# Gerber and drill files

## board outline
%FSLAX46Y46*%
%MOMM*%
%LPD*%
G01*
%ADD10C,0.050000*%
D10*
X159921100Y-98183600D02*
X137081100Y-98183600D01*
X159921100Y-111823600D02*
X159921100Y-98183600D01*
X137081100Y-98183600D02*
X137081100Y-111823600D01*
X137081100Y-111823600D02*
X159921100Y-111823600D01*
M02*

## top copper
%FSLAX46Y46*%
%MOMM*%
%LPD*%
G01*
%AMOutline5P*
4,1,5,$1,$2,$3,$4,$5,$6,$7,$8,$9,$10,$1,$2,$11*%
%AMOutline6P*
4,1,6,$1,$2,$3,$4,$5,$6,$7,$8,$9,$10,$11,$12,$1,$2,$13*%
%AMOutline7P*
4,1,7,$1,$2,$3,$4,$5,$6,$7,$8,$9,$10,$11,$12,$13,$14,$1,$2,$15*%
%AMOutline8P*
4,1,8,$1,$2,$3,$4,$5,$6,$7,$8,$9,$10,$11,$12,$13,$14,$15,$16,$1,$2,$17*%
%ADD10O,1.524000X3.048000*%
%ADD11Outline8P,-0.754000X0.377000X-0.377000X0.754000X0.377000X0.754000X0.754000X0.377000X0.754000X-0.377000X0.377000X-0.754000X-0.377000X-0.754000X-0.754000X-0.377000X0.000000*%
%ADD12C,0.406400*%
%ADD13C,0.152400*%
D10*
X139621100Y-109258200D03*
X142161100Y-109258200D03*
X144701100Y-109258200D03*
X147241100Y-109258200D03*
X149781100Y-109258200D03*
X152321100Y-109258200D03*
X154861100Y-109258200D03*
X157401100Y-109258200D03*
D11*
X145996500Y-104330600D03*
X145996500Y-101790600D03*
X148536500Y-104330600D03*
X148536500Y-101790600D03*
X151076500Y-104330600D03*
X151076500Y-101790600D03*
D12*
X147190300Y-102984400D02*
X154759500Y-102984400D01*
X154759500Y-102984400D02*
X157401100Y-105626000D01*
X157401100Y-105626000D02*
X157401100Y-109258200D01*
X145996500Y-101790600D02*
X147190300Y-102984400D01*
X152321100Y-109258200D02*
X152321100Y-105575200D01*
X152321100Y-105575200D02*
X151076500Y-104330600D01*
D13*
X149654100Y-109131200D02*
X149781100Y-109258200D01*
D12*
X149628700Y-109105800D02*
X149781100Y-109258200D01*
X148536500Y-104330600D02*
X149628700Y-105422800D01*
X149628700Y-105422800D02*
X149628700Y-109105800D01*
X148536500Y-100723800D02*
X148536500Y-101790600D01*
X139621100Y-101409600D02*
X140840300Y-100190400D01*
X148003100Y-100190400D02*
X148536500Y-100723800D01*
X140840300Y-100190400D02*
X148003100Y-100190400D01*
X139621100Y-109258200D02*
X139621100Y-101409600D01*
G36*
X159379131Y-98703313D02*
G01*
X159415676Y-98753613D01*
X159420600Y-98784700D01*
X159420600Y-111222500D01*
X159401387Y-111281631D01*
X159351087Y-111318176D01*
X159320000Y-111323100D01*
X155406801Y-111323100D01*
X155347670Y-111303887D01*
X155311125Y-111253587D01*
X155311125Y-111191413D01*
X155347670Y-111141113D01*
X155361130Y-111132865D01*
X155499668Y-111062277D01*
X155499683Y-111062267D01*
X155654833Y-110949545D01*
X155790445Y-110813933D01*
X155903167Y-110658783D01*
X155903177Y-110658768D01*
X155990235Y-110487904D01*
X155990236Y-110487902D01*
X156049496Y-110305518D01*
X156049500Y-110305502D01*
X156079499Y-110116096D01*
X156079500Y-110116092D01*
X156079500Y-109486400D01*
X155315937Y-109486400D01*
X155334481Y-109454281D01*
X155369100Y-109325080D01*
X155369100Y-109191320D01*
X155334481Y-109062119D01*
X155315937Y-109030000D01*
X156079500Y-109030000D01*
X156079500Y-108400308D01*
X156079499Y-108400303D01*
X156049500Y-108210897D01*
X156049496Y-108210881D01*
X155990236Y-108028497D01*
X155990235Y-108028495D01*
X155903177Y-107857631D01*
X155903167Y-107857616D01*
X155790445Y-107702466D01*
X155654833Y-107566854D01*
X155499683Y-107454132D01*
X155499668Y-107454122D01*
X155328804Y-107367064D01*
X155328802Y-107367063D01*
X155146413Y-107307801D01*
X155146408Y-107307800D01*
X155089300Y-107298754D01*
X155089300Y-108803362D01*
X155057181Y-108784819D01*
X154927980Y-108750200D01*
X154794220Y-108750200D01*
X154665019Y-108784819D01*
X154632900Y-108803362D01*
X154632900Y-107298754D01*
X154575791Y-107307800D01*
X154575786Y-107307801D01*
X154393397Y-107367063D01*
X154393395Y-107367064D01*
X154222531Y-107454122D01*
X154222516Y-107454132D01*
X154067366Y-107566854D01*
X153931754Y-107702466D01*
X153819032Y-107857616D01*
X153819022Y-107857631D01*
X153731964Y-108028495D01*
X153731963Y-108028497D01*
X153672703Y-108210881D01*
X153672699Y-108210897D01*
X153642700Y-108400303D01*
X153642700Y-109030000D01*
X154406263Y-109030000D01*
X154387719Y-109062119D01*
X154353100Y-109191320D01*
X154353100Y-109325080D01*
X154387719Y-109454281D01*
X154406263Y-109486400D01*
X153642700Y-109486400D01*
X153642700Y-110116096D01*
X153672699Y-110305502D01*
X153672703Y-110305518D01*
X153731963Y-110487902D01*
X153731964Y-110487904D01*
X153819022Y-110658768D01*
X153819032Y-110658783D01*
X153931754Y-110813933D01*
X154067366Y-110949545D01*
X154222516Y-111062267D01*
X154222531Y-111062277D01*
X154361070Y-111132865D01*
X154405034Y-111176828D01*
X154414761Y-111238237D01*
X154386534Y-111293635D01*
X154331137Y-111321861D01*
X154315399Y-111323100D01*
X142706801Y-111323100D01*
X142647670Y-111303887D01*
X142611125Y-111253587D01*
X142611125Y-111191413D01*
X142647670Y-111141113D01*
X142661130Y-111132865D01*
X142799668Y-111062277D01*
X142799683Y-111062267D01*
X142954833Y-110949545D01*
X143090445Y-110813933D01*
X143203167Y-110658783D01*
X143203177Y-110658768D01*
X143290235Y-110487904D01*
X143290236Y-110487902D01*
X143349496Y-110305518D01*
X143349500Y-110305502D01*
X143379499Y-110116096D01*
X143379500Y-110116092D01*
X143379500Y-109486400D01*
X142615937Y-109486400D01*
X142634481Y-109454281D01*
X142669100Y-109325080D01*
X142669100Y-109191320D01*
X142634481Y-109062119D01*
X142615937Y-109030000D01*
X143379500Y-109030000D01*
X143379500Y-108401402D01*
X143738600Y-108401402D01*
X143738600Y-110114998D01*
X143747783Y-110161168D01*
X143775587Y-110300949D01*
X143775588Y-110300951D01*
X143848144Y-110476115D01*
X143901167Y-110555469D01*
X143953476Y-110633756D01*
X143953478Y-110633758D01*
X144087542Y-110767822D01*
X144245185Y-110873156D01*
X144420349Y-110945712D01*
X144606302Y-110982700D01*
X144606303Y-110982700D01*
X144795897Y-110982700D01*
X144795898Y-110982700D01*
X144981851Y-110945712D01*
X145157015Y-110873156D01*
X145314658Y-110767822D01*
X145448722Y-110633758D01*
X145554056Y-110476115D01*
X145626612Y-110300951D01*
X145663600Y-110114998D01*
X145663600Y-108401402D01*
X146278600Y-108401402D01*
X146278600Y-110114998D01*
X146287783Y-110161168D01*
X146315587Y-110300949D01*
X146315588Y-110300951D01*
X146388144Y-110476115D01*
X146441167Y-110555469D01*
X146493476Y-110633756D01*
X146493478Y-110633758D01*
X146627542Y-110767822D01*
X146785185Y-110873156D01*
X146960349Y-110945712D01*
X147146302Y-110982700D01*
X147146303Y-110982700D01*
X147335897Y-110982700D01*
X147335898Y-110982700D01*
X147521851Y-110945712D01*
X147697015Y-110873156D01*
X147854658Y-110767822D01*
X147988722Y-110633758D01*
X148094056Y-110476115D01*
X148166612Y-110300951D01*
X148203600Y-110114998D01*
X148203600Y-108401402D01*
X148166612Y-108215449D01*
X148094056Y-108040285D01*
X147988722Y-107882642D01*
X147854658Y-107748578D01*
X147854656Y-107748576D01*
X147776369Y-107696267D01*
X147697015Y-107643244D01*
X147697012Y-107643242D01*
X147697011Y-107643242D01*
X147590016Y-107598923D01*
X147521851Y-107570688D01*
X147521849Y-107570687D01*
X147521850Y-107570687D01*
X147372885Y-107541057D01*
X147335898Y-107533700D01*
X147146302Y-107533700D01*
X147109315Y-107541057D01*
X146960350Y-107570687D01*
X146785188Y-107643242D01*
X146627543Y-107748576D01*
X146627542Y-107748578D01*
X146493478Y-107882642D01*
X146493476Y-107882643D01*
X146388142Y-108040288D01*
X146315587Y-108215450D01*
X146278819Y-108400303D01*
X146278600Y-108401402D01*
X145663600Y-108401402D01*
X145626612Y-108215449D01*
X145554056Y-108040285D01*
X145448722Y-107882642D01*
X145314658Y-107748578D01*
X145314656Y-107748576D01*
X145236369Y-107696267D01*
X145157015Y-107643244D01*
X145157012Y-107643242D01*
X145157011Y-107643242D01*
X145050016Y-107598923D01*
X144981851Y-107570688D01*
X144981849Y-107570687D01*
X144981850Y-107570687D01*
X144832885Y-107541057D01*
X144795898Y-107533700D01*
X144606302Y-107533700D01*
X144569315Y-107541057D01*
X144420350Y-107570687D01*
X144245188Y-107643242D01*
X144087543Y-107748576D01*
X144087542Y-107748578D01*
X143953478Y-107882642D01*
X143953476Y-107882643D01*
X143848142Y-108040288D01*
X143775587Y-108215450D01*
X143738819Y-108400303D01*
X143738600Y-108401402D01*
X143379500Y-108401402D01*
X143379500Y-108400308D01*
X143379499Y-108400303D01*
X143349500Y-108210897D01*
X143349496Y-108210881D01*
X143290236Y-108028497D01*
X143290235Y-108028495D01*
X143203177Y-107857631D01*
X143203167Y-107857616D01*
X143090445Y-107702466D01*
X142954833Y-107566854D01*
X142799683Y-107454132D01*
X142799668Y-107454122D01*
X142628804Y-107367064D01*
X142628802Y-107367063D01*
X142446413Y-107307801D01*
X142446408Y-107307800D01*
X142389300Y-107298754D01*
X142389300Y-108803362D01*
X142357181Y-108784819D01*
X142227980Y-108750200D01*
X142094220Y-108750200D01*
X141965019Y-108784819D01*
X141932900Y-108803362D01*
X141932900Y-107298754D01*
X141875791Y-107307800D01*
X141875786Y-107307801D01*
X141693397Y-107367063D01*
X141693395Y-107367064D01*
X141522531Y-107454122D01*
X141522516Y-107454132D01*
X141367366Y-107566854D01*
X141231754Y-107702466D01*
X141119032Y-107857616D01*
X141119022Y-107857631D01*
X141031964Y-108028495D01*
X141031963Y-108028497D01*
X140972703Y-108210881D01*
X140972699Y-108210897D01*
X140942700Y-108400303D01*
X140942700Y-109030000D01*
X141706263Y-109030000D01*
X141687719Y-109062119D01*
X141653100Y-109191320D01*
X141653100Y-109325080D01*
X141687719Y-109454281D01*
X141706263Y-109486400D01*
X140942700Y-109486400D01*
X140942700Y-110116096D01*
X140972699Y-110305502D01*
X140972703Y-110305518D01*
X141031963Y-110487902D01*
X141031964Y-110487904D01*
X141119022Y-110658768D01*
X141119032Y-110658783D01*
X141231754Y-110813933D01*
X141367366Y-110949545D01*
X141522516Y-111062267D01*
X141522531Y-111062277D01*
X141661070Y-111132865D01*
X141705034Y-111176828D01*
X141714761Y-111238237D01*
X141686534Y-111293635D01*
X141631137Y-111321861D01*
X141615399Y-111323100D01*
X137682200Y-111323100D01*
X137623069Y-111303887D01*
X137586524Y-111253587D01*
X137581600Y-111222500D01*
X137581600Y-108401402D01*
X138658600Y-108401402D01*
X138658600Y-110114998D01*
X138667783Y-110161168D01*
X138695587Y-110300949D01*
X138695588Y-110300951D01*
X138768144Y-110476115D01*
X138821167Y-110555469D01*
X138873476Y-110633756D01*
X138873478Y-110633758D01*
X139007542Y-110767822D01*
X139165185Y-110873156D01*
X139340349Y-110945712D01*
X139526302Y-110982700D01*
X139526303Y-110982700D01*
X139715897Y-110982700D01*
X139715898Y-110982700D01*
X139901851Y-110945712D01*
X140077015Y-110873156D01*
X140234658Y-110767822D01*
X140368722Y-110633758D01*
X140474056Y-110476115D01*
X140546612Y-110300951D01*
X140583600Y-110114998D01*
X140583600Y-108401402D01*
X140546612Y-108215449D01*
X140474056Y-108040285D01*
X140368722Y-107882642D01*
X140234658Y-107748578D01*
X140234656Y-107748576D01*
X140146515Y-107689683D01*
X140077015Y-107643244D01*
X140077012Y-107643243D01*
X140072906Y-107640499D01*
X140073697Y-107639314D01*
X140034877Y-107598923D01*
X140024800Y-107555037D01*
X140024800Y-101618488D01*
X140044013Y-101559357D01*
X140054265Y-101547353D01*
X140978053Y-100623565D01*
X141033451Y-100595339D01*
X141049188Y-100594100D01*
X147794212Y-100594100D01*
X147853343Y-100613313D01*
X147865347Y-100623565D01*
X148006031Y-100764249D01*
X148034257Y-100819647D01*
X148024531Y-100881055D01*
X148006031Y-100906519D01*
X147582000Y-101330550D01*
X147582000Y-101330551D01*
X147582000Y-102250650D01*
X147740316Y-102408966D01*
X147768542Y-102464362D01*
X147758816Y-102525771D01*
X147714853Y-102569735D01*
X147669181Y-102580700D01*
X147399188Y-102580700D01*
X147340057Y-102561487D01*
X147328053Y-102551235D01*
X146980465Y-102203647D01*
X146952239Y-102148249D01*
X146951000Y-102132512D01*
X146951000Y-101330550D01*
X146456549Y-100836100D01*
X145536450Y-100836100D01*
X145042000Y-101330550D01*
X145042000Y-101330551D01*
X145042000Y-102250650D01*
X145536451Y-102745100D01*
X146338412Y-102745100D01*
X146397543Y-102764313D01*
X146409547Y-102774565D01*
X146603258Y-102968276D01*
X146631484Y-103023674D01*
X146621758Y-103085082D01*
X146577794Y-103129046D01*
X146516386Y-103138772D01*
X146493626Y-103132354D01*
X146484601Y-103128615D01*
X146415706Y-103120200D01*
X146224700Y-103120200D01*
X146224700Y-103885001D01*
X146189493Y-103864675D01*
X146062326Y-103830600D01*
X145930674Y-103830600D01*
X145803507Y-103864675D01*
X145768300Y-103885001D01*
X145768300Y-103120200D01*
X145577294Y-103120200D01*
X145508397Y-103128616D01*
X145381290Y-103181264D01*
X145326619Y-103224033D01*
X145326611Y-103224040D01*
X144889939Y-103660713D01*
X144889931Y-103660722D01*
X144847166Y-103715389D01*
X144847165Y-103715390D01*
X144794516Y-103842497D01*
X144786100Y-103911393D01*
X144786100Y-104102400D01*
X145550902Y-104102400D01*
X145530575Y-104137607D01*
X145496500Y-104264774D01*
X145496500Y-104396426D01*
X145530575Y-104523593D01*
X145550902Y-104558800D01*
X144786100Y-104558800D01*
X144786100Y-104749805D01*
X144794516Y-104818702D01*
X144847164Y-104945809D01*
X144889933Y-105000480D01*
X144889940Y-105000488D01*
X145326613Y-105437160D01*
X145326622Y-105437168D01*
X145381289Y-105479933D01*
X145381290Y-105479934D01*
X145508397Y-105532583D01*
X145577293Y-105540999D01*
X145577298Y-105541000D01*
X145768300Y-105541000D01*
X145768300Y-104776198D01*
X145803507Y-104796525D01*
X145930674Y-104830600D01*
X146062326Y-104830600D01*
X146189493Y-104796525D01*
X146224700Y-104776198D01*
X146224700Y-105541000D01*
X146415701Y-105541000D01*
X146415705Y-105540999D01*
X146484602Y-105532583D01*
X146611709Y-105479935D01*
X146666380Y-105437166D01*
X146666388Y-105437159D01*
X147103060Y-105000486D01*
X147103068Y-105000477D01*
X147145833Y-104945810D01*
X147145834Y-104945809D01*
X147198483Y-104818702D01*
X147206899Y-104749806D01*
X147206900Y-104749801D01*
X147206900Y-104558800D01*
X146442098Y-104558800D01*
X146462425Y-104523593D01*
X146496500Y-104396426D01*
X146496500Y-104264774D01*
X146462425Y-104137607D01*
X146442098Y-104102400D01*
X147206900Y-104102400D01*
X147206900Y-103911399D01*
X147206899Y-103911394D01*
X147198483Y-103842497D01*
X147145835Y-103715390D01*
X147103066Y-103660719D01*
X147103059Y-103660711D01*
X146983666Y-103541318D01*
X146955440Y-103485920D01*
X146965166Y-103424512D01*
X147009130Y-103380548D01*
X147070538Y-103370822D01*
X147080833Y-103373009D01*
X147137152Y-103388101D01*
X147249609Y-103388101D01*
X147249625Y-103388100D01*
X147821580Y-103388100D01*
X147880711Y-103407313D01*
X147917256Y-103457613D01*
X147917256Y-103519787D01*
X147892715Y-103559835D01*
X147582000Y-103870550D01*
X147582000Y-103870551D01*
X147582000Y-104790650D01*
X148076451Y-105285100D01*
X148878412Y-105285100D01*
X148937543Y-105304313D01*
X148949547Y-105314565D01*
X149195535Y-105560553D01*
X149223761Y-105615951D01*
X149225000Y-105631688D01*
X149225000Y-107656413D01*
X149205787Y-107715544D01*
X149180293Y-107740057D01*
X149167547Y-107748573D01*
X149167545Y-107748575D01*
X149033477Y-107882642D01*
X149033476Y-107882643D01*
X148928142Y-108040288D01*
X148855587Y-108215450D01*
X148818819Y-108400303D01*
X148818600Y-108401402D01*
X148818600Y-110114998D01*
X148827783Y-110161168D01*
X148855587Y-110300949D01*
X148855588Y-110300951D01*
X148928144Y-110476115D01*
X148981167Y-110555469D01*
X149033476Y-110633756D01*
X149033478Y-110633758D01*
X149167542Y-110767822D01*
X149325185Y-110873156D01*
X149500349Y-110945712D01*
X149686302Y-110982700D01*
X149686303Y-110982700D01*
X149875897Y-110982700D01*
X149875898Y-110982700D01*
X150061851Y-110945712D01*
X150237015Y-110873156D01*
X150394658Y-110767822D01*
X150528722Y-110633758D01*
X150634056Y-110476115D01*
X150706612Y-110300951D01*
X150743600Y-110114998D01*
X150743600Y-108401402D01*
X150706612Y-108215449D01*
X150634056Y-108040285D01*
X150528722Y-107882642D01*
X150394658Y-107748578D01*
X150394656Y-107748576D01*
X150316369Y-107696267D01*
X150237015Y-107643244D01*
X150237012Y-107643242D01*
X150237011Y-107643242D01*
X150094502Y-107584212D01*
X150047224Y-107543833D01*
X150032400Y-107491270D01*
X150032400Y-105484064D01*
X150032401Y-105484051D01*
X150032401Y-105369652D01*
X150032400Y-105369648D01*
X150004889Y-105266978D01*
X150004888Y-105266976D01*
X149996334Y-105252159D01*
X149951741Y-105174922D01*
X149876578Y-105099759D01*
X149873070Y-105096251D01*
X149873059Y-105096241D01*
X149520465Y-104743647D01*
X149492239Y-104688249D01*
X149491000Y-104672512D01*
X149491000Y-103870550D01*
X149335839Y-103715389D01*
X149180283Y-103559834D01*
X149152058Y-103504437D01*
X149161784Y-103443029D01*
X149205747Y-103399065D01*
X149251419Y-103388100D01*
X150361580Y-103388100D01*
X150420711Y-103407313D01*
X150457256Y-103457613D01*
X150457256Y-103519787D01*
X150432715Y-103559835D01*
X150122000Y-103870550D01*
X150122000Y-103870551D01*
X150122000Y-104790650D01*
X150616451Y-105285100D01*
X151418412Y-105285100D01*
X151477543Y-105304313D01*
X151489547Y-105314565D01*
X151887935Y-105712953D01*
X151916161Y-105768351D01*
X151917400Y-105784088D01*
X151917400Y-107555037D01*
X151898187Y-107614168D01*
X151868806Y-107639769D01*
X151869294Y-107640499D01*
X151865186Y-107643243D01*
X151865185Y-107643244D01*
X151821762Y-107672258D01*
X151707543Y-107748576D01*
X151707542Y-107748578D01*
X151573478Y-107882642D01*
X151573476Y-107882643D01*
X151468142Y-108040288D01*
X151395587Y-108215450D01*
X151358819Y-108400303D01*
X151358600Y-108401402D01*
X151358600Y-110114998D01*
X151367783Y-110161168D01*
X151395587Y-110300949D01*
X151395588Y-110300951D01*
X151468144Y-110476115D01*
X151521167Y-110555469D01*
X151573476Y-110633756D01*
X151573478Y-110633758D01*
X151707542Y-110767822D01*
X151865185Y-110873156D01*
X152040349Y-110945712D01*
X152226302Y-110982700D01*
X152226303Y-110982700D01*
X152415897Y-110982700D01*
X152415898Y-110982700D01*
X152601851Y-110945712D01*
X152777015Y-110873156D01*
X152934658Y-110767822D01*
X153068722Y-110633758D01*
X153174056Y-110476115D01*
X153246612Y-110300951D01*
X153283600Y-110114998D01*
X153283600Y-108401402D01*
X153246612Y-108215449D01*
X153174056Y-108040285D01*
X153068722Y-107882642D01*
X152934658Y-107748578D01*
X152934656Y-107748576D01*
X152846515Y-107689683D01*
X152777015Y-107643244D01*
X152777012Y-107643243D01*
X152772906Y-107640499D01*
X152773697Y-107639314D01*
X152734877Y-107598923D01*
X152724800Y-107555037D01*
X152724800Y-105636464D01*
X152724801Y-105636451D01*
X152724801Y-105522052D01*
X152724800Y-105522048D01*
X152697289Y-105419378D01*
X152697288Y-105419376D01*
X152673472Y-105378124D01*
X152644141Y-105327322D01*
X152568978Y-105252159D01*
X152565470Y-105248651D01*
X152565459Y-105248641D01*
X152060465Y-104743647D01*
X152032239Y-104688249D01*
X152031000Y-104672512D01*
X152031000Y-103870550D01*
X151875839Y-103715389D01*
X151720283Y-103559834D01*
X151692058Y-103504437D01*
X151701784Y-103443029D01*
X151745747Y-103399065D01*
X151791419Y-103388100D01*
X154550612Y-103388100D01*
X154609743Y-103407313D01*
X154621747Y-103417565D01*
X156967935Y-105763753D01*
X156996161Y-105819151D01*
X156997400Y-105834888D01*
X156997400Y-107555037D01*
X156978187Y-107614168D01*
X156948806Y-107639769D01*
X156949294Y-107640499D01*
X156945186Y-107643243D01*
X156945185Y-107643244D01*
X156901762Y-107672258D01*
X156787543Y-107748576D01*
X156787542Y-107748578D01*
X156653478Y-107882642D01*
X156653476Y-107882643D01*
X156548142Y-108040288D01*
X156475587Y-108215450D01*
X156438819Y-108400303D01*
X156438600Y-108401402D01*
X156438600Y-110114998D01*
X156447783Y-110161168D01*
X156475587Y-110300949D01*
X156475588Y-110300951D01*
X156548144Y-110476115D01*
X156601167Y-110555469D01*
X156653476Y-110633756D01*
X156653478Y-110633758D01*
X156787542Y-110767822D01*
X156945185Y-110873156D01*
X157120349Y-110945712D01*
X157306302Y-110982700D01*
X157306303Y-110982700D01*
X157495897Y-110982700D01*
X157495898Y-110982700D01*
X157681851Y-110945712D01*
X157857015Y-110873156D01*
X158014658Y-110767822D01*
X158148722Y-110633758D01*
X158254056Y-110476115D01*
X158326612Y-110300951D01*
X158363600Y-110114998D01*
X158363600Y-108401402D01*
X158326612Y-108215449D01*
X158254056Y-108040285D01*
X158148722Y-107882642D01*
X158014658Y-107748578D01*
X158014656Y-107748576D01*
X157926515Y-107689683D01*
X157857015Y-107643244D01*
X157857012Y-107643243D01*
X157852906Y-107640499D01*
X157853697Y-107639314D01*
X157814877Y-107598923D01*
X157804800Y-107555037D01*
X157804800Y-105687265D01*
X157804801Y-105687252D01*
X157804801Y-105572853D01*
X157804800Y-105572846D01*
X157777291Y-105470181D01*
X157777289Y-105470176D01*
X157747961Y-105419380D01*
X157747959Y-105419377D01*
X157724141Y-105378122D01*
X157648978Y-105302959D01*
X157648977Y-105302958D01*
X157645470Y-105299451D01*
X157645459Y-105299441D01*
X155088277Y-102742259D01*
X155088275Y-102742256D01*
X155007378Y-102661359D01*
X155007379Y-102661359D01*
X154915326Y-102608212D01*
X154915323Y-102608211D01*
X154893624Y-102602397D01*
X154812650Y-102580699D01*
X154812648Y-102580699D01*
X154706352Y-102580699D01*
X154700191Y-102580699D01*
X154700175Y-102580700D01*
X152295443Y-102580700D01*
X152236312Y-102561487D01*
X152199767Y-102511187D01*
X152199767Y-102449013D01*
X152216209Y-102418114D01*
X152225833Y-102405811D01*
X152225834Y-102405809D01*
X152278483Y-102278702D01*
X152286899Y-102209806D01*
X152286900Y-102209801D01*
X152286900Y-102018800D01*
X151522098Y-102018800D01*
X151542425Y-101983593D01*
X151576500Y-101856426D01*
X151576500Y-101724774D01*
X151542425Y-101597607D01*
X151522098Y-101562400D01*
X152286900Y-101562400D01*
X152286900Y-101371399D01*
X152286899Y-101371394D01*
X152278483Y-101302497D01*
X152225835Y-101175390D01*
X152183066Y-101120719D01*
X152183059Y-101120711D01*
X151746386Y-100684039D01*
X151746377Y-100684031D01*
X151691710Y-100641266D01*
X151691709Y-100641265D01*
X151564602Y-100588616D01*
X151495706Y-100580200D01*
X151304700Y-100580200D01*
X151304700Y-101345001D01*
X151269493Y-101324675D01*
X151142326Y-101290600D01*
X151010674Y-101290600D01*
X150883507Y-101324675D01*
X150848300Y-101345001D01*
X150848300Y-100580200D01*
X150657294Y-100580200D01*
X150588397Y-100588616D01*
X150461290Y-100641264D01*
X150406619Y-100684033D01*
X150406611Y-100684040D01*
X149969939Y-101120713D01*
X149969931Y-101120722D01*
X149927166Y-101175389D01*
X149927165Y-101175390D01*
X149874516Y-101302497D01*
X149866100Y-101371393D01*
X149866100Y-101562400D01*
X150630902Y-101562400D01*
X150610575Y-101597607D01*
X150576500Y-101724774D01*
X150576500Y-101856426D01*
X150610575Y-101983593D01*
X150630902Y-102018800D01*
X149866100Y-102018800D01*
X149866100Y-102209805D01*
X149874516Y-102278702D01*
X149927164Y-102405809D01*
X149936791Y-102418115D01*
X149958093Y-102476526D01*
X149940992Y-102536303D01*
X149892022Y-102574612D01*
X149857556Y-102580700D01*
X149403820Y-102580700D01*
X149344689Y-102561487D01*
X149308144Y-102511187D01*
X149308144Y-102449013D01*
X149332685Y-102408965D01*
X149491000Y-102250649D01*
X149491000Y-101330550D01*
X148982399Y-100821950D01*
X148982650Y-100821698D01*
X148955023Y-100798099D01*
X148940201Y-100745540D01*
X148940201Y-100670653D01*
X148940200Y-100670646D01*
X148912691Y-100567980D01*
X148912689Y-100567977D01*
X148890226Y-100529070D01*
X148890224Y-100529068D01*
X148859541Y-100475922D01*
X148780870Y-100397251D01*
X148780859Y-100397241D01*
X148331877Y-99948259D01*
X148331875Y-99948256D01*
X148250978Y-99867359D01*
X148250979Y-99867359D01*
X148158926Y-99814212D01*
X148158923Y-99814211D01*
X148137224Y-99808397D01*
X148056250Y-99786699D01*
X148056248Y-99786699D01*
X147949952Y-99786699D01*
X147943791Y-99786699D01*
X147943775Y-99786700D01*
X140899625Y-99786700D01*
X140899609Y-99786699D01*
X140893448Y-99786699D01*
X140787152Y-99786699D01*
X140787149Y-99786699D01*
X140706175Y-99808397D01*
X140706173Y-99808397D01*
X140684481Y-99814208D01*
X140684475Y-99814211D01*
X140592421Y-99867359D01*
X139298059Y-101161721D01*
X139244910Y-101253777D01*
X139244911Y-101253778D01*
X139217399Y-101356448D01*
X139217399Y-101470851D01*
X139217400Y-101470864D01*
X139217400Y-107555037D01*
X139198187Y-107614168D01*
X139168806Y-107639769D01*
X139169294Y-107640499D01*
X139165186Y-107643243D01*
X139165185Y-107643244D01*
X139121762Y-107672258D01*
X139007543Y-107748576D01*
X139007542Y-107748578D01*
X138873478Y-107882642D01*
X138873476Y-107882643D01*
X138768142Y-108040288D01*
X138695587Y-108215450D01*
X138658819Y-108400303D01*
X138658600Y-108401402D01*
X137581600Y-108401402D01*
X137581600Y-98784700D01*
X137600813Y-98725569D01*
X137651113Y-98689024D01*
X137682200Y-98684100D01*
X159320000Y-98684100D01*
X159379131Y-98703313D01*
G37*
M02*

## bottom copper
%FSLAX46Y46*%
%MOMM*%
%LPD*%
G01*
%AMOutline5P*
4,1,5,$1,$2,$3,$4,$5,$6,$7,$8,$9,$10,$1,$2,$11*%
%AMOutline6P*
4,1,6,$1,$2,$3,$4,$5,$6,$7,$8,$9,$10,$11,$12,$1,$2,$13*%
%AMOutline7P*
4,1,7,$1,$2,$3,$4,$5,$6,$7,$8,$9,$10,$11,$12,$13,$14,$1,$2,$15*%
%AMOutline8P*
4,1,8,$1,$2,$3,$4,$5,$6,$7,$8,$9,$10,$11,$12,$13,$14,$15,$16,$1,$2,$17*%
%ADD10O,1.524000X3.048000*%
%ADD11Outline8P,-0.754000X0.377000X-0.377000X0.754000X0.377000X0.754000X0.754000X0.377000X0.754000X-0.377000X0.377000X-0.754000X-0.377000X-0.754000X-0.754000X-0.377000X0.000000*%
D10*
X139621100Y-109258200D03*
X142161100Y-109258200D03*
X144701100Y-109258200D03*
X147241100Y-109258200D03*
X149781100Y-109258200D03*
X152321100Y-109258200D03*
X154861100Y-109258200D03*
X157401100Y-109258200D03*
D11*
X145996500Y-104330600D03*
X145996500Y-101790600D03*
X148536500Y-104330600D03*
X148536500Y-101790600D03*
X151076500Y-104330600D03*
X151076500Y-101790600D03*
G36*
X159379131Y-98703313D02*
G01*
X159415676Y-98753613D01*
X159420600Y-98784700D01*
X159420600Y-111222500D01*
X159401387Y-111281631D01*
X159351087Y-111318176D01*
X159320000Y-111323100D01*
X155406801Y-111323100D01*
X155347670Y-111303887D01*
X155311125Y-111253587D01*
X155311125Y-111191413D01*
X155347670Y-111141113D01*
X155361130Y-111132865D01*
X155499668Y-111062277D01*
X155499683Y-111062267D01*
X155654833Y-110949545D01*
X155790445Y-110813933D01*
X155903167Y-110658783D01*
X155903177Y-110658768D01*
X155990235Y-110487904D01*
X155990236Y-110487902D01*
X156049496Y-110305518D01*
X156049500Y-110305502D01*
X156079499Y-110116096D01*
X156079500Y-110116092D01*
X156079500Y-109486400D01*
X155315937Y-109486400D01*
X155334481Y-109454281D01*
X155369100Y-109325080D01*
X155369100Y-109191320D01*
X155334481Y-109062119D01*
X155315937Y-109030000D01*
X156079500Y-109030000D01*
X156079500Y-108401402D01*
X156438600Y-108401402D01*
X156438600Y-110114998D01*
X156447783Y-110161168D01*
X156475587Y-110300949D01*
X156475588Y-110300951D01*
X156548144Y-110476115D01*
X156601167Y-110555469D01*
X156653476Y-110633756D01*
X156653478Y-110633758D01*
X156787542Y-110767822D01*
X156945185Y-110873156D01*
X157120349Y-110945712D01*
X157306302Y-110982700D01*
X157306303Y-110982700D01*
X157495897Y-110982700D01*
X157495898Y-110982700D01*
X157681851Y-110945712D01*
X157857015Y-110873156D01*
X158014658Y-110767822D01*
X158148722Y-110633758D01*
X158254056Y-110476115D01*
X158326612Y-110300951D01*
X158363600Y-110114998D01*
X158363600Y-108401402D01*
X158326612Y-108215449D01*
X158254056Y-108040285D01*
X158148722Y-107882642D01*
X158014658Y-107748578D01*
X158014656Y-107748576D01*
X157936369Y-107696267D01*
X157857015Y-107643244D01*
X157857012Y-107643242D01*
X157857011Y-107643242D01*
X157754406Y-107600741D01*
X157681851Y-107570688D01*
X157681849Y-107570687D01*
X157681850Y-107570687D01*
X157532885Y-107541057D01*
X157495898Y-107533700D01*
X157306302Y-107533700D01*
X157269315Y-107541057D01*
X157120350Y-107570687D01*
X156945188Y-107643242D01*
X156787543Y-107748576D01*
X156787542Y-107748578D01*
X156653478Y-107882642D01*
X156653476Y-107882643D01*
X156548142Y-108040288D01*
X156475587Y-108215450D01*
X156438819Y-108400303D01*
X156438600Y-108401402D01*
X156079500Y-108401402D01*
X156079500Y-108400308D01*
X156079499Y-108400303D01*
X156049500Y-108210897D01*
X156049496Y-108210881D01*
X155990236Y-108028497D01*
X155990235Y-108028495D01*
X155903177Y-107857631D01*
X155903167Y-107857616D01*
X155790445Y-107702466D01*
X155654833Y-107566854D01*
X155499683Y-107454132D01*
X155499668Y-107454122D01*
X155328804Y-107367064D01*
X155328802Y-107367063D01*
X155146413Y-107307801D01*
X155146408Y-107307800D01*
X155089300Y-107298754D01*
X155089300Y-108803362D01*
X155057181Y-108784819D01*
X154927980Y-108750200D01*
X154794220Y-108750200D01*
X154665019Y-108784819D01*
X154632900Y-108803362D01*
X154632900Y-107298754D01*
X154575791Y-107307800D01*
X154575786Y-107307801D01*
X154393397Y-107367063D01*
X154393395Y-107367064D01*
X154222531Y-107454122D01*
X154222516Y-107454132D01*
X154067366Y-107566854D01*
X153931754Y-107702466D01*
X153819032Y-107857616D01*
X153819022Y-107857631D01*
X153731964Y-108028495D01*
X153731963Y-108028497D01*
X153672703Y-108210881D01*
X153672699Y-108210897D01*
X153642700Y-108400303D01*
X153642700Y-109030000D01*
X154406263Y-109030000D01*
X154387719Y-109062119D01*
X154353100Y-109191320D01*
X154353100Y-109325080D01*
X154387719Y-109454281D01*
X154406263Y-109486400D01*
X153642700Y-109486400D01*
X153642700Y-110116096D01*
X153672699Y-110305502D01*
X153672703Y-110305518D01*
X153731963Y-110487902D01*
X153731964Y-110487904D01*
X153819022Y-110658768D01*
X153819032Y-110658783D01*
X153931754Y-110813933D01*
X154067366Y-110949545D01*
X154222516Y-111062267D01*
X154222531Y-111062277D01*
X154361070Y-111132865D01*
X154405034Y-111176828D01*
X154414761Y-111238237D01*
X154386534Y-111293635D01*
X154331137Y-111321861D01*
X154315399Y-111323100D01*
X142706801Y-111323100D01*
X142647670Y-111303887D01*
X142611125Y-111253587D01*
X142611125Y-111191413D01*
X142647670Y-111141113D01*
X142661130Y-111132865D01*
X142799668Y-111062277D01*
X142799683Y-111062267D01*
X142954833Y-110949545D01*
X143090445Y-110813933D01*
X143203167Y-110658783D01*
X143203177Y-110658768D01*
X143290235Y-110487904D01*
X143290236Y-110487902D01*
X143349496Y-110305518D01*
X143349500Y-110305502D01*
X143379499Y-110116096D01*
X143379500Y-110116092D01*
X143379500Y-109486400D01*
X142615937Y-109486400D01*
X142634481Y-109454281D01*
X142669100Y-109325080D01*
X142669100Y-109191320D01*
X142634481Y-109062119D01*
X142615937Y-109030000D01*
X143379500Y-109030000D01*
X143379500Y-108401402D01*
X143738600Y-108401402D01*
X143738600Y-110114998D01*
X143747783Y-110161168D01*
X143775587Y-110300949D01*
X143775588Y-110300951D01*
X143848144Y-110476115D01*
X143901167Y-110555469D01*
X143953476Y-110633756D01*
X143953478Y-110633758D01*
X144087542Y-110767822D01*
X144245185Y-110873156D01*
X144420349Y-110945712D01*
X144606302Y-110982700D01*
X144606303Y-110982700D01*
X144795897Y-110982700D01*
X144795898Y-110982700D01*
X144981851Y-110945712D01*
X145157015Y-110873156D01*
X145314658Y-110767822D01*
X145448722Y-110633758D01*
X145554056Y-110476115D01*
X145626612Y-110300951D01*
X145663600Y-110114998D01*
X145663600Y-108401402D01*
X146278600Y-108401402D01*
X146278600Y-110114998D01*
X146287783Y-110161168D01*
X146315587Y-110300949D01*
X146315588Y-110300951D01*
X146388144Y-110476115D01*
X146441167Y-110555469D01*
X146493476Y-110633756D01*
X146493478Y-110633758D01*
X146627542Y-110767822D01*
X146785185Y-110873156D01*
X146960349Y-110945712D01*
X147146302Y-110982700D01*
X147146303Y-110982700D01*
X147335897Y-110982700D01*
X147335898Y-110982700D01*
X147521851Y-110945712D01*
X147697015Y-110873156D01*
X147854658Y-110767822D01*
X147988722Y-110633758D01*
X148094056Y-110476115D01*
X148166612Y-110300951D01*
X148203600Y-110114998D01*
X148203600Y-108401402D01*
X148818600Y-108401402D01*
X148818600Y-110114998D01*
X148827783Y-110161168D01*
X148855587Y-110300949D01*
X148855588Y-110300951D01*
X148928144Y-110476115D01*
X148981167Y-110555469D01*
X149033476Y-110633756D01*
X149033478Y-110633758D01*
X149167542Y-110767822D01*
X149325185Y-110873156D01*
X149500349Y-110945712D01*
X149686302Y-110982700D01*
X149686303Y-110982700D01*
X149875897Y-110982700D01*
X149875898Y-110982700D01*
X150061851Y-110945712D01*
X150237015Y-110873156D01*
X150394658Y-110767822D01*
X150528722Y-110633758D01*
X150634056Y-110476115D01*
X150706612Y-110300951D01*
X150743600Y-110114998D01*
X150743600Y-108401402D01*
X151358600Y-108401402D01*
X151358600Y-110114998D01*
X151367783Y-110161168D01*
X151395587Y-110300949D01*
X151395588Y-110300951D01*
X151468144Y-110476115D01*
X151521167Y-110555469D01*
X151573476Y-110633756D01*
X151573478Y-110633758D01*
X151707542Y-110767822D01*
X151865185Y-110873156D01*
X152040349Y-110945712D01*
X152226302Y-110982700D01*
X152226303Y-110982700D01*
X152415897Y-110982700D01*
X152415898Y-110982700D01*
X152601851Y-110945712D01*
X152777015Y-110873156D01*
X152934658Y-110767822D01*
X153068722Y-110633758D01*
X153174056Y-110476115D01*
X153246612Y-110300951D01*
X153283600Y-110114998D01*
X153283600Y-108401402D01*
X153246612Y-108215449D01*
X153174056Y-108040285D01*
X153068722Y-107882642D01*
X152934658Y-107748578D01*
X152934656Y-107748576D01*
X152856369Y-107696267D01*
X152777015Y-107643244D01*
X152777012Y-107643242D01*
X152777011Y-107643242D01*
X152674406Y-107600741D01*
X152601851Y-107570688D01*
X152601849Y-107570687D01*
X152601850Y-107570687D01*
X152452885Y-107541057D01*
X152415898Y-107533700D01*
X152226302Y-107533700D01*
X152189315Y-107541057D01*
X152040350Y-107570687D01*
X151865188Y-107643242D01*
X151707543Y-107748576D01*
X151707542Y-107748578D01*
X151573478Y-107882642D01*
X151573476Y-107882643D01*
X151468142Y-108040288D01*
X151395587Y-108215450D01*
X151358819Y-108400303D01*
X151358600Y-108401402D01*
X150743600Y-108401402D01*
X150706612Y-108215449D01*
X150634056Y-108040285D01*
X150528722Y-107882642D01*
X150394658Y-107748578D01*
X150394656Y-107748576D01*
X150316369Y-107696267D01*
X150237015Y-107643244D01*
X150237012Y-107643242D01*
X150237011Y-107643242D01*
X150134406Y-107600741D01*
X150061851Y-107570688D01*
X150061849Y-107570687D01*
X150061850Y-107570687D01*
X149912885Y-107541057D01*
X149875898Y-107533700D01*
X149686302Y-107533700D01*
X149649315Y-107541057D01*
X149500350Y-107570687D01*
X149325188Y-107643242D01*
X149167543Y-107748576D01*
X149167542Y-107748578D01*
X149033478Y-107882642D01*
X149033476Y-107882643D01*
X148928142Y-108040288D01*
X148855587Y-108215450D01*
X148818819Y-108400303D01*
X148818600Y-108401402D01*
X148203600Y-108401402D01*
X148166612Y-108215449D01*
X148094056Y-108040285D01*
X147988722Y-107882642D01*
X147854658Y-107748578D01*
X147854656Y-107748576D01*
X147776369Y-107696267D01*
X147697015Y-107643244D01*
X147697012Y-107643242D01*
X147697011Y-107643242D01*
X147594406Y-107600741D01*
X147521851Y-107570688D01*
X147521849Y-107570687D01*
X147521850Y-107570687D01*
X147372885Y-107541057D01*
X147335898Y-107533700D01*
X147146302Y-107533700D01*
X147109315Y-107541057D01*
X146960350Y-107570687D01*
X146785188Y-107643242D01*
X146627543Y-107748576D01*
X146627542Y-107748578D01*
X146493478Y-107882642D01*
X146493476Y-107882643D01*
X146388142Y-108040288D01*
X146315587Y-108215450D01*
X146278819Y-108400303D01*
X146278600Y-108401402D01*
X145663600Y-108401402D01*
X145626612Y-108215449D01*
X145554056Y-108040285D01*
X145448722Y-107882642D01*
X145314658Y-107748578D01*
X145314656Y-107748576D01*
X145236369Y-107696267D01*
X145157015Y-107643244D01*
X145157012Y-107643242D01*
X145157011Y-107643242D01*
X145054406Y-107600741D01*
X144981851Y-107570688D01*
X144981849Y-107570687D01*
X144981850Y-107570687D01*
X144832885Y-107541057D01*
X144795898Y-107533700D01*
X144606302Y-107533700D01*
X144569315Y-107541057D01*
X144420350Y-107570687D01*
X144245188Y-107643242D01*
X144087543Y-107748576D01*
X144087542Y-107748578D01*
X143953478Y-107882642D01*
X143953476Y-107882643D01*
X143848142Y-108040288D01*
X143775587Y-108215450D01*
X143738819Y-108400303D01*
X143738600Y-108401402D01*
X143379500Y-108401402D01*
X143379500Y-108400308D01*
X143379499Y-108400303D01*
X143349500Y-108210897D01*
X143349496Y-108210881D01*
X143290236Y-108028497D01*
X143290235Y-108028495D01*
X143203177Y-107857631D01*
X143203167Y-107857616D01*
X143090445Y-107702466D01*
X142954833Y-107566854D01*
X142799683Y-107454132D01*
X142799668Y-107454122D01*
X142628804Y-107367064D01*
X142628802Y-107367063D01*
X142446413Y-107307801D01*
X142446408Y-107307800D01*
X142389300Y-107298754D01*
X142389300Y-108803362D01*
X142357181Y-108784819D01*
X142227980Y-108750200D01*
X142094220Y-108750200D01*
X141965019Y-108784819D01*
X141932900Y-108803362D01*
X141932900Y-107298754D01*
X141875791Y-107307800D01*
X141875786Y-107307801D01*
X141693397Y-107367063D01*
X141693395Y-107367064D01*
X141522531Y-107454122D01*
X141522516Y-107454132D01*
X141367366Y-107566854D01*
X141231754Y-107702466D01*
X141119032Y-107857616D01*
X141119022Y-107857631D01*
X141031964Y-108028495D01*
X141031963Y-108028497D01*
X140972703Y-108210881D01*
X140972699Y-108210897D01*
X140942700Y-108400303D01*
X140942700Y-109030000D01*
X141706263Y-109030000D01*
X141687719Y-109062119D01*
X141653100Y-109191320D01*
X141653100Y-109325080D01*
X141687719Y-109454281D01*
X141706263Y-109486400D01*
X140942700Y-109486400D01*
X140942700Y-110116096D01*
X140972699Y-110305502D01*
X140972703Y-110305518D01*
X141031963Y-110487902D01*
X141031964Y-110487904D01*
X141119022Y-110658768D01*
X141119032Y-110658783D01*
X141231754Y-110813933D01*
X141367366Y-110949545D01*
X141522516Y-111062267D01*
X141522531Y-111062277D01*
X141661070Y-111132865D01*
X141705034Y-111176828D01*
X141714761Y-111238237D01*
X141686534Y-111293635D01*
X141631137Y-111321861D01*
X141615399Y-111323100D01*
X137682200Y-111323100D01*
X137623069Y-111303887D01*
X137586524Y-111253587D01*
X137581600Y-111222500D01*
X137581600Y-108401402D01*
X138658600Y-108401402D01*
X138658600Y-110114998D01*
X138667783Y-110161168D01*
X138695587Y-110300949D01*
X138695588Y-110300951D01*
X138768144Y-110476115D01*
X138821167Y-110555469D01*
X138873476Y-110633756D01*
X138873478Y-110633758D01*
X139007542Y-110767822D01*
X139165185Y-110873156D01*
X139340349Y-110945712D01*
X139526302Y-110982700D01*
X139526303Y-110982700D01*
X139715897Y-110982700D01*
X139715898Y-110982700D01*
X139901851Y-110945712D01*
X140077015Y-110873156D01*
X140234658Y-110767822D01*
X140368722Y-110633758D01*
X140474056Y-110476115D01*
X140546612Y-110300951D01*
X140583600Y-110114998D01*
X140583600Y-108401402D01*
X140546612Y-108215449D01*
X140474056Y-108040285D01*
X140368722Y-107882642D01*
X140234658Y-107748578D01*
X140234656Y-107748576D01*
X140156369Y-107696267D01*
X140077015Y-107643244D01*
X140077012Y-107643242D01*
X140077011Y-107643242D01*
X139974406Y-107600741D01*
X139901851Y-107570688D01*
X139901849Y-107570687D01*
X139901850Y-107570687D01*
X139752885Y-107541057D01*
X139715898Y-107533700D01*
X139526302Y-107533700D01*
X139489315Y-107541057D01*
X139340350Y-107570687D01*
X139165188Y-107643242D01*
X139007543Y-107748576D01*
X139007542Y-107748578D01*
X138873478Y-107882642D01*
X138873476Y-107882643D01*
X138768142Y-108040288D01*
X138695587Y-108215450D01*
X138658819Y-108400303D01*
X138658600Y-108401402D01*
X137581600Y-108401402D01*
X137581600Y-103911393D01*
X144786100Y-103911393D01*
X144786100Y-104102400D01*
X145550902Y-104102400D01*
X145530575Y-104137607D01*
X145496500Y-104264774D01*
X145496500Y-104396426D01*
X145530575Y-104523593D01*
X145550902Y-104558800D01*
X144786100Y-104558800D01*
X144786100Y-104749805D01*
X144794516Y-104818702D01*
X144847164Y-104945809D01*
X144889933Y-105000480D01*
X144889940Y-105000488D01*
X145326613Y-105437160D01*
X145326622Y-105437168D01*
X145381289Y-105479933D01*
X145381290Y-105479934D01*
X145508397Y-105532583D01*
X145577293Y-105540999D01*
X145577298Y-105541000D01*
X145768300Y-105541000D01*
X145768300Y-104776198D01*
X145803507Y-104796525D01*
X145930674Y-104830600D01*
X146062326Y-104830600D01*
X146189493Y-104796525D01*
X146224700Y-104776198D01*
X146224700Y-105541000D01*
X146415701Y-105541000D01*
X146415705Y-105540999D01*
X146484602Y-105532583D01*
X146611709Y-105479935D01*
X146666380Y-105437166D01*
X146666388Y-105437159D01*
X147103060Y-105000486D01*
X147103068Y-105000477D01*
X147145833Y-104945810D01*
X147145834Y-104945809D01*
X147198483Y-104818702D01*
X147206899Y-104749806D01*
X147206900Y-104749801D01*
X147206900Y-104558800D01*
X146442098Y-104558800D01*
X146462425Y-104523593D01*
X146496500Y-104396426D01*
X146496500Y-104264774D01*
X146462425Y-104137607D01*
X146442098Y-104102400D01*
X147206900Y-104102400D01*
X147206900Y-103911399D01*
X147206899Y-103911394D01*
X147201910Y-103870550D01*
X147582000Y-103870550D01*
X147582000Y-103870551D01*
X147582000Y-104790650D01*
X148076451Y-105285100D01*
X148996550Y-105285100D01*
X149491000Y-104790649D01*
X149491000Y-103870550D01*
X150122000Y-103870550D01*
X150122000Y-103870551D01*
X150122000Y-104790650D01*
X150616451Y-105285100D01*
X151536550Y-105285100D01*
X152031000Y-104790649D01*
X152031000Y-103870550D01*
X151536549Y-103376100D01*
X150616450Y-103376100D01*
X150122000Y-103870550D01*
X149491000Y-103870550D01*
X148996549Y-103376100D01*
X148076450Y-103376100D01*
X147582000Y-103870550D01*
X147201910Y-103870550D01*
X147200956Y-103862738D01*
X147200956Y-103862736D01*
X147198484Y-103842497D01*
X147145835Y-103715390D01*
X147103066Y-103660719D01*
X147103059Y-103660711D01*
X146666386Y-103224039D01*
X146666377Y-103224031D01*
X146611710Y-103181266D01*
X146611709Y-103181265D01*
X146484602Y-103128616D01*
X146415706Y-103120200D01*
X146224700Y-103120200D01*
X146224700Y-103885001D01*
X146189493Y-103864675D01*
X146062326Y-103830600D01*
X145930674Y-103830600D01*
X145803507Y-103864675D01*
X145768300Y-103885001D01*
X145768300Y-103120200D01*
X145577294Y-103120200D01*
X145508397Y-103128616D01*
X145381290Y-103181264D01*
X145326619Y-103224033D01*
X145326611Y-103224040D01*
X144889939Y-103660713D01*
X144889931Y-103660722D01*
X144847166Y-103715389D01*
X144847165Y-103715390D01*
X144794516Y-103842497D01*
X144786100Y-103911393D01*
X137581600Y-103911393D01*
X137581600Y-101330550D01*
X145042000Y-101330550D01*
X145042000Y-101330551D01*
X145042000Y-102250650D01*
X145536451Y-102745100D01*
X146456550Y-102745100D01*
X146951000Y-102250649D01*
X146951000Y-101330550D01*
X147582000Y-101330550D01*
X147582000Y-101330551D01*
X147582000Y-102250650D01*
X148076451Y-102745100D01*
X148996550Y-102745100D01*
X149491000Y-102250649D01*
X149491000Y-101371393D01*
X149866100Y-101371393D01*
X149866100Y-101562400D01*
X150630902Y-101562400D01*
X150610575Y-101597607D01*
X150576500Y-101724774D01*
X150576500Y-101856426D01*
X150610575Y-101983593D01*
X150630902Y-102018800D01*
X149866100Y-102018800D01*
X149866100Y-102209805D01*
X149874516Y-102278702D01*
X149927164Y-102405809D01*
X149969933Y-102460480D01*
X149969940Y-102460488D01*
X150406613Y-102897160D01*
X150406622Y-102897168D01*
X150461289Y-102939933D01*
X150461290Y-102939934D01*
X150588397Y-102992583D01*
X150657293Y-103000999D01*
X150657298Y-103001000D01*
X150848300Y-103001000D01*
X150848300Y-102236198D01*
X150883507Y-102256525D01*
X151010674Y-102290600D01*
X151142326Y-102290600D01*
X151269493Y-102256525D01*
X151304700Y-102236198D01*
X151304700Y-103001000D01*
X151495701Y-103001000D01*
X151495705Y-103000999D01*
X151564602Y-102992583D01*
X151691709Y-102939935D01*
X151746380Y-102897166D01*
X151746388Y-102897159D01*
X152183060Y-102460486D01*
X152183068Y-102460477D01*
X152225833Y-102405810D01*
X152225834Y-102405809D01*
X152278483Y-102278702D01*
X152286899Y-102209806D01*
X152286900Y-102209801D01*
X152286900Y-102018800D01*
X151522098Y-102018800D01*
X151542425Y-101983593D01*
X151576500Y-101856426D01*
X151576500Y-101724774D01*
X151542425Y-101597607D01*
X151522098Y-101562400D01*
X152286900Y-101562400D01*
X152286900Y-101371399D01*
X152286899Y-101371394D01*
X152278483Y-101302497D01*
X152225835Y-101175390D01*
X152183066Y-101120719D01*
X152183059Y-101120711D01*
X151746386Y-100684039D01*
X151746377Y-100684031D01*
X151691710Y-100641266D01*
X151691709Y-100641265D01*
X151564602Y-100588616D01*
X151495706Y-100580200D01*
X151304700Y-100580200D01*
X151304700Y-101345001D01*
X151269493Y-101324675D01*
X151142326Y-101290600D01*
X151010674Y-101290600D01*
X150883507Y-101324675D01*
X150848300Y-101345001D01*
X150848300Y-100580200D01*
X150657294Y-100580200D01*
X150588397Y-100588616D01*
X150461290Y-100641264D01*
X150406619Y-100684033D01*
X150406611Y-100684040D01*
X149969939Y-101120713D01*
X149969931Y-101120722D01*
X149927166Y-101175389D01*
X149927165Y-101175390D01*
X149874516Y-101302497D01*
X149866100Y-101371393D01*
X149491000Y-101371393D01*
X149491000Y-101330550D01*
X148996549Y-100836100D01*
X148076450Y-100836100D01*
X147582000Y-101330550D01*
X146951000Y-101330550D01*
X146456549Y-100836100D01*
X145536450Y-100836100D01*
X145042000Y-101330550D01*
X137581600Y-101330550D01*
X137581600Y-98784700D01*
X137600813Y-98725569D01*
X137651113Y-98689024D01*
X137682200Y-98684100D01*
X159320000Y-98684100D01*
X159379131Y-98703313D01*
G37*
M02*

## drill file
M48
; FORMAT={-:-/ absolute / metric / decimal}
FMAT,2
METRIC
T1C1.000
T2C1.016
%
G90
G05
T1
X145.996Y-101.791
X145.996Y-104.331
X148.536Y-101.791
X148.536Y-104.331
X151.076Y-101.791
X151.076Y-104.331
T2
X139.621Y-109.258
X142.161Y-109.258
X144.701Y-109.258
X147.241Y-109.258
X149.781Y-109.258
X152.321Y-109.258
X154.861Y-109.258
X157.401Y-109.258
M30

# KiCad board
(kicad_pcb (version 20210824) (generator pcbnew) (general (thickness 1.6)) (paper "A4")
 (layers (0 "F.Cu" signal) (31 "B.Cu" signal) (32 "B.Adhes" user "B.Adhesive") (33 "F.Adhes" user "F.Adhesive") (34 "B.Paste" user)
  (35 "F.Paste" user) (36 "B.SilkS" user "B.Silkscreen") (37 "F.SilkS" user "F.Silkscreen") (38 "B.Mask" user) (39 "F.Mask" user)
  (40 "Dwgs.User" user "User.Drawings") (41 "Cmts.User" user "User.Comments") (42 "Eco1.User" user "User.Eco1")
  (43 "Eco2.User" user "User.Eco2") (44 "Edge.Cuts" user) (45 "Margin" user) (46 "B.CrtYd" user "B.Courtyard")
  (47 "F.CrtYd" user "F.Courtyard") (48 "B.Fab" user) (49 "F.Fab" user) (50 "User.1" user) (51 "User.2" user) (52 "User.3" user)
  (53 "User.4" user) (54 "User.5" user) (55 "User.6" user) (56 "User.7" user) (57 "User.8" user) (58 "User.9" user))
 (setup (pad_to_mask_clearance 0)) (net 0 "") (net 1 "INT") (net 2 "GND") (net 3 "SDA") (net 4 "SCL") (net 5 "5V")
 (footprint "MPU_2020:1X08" (layer "F.Cu") (at 148.5111 109.2582)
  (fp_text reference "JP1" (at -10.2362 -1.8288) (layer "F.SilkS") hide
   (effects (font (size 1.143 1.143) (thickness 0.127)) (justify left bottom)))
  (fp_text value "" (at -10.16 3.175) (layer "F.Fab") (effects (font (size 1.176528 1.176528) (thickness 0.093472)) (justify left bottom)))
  (pad "1" thru_hole oval (at -8.89 0 90) (size 3.048 1.524) (drill 1.016) (layers *.Cu *.Mask) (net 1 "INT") (solder_mask_margin 0.1016))
  (pad "2" thru_hole oval (at -6.35 0 90) (size 3.048 1.524) (drill 1.016) (layers *.Cu *.Mask) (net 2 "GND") (solder_mask_margin 0.1016))
  (pad "3" thru_hole oval (at -3.81 0 90) (size 3.048 1.524) (drill 1.016) (layers *.Cu *.Mask) (solder_mask_margin 0.1016))
  (pad "4" thru_hole oval (at -1.27 0 90) (size 3.048 1.524) (drill 1.016) (layers *.Cu *.Mask) (solder_mask_margin 0.1016))
  (pad "5" thru_hole oval (at 1.27 0 90) (size 3.048 1.524) (drill 1.016) (layers *.Cu *.Mask) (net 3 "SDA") (solder_mask_margin 0.1016))
  (pad "6" thru_hole oval (at 3.81 0 90) (size 3.048 1.524) (drill 1.016) (layers *.Cu *.Mask) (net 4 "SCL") (solder_mask_margin 0.1016))
  (pad "7" thru_hole oval (at 6.35 0 90) (size 3.048 1.524) (drill 1.016) (layers *.Cu *.Mask) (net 2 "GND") (solder_mask_margin 0.1016))
  (pad "8" thru_hole oval (at 8.89 0 90) (size 3.048 1.524) (drill 1.016) (layers *.Cu *.Mask) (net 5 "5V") (solder_mask_margin 0.1016)))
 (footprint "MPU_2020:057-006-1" (layer "F.Cu") (at 148.5365 103.0606)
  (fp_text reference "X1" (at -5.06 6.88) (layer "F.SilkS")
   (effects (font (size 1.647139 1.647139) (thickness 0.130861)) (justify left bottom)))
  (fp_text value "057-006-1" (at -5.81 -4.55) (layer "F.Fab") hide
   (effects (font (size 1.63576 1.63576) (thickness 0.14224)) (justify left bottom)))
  (pad "1" thru_hole roundrect (at -2.54 1.27) (size 1.508 1.508) (drill 1) (layers *.Cu *.Mask) (roundrect_rratio 0.25)
   (chamfer_ratio 0.25) (chamfer top_left top_right bottom_left bottom_right) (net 2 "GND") (solder_mask_margin 0.1016))
  (pad "2" thru_hole roundrect (at -2.54 -1.27) (size 1.508 1.508) (drill 1) (layers *.Cu *.Mask) (roundrect_rratio 0.25)
   (chamfer_ratio 0.25) (chamfer top_left top_right bottom_left bottom_right) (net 5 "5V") (solder_mask_margin 0.1016))
  (pad "3" thru_hole roundrect (at 0 1.27) (size 1.508 1.508) (drill 1) (layers *.Cu *.Mask) (roundrect_rratio 0.25) (chamfer_ratio 0.25)
   (chamfer top_left top_right bottom_left bottom_right) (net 3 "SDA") (solder_mask_margin 0.1016))
  (pad "4" thru_hole roundrect (at 0 -1.27) (size 1.508 1.508) (drill 1) (layers *.Cu *.Mask) (roundrect_rratio 0.25) (chamfer_ratio 0.25)
   (chamfer top_left top_right bottom_left bottom_right) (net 1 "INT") (solder_mask_margin 0.1016))
  (pad "5" thru_hole roundrect (at 2.54 1.27) (size 1.508 1.508) (drill 1) (layers *.Cu *.Mask) (roundrect_rratio 0.25) (chamfer_ratio 0.25)
   (chamfer top_left top_right bottom_left bottom_right) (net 4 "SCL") (solder_mask_margin 0.1016))
  (pad "6" thru_hole roundrect (at 2.54 -1.27) (size 1.508 1.508) (drill 1) (layers *.Cu *.Mask) (roundrect_rratio 0.25)
   (chamfer_ratio 0.25) (chamfer top_left top_right bottom_left bottom_right) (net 2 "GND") (solder_mask_margin 0.1016)))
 (gr_line (start 159.9211 98.1836) (end 137.0811 98.1836) (layer "Edge.Cuts") (width 0.05))
 (gr_line (start 159.9211 111.8236) (end 159.9211 98.1836) (layer "Edge.Cuts") (width 0.05))
 (gr_line (start 137.0811 98.1836) (end 137.0811 111.8236) (layer "Edge.Cuts") (width 0.05))
 (gr_line (start 137.0811 111.8236) (end 159.9211 111.8236) (layer "Edge.Cuts") (width 0.05))
 (segment (start 147.1903 102.9844) (end 154.7595 102.9844) (width 0.4064) (layer "F.Cu") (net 5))
 (segment (start 154.7595 102.9844) (end 157.4011 105.626) (width 0.4064) (layer "F.Cu") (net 5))
 (segment (start 157.4011 105.626) (end 157.4011 109.2582) (width 0.4064) (layer "F.Cu") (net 5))
 (segment (start 145.9965 101.7906) (end 147.1903 102.9844) (width 0.4064) (layer "F.Cu") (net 5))
 (segment (start 152.3211 109.2582) (end 152.3211 105.5752) (width 0.4064) (layer "F.Cu") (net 4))
 (segment (start 152.3211 105.5752) (end 151.0765 104.3306) (width 0.4064) (layer "F.Cu") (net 4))
 (segment (start 149.6541 109.1312) (end 149.7811 109.2582) (width 0.1524) (layer "F.Cu") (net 3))
 (segment (start 149.6287 109.1058) (end 149.7811 109.2582) (width 0.4064) (layer "F.Cu") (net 3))
 (segment (start 148.5365 104.3306) (end 149.6287 105.4228) (width 0.4064) (layer "F.Cu") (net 3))
 (segment (start 149.6287 105.4228) (end 149.6287 109.1058) (width 0.4064) (layer "F.Cu") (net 3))
 (segment (start 148.5365 100.7238) (end 148.5365 101.7906) (width 0.4064) (layer "F.Cu") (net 1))
 (segment (start 139.6211 101.4096) (end 140.8403 100.1904) (width 0.4064) (layer "F.Cu") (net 1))
 (segment (start 148.0031 100.1904) (end 148.5365 100.7238) (width 0.4064) (layer "F.Cu") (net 1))
 (segment (start 140.8403 100.1904) (end 148.0031 100.1904) (width 0.4064) (layer "F.Cu") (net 1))
 (segment (start 139.6211 109.2582) (end 139.6211 101.4096) (width 0.4064) (layer "F.Cu") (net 1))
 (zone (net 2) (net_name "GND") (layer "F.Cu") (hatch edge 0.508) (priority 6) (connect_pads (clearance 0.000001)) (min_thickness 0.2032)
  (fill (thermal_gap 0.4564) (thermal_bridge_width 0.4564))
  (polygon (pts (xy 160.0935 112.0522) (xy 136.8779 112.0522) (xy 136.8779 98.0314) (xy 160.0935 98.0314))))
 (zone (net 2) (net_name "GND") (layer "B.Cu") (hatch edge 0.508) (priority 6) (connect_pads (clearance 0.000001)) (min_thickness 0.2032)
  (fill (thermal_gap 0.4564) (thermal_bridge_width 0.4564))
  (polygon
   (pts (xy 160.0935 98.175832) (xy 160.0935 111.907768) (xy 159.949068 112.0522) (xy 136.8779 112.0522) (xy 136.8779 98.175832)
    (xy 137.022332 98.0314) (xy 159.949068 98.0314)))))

